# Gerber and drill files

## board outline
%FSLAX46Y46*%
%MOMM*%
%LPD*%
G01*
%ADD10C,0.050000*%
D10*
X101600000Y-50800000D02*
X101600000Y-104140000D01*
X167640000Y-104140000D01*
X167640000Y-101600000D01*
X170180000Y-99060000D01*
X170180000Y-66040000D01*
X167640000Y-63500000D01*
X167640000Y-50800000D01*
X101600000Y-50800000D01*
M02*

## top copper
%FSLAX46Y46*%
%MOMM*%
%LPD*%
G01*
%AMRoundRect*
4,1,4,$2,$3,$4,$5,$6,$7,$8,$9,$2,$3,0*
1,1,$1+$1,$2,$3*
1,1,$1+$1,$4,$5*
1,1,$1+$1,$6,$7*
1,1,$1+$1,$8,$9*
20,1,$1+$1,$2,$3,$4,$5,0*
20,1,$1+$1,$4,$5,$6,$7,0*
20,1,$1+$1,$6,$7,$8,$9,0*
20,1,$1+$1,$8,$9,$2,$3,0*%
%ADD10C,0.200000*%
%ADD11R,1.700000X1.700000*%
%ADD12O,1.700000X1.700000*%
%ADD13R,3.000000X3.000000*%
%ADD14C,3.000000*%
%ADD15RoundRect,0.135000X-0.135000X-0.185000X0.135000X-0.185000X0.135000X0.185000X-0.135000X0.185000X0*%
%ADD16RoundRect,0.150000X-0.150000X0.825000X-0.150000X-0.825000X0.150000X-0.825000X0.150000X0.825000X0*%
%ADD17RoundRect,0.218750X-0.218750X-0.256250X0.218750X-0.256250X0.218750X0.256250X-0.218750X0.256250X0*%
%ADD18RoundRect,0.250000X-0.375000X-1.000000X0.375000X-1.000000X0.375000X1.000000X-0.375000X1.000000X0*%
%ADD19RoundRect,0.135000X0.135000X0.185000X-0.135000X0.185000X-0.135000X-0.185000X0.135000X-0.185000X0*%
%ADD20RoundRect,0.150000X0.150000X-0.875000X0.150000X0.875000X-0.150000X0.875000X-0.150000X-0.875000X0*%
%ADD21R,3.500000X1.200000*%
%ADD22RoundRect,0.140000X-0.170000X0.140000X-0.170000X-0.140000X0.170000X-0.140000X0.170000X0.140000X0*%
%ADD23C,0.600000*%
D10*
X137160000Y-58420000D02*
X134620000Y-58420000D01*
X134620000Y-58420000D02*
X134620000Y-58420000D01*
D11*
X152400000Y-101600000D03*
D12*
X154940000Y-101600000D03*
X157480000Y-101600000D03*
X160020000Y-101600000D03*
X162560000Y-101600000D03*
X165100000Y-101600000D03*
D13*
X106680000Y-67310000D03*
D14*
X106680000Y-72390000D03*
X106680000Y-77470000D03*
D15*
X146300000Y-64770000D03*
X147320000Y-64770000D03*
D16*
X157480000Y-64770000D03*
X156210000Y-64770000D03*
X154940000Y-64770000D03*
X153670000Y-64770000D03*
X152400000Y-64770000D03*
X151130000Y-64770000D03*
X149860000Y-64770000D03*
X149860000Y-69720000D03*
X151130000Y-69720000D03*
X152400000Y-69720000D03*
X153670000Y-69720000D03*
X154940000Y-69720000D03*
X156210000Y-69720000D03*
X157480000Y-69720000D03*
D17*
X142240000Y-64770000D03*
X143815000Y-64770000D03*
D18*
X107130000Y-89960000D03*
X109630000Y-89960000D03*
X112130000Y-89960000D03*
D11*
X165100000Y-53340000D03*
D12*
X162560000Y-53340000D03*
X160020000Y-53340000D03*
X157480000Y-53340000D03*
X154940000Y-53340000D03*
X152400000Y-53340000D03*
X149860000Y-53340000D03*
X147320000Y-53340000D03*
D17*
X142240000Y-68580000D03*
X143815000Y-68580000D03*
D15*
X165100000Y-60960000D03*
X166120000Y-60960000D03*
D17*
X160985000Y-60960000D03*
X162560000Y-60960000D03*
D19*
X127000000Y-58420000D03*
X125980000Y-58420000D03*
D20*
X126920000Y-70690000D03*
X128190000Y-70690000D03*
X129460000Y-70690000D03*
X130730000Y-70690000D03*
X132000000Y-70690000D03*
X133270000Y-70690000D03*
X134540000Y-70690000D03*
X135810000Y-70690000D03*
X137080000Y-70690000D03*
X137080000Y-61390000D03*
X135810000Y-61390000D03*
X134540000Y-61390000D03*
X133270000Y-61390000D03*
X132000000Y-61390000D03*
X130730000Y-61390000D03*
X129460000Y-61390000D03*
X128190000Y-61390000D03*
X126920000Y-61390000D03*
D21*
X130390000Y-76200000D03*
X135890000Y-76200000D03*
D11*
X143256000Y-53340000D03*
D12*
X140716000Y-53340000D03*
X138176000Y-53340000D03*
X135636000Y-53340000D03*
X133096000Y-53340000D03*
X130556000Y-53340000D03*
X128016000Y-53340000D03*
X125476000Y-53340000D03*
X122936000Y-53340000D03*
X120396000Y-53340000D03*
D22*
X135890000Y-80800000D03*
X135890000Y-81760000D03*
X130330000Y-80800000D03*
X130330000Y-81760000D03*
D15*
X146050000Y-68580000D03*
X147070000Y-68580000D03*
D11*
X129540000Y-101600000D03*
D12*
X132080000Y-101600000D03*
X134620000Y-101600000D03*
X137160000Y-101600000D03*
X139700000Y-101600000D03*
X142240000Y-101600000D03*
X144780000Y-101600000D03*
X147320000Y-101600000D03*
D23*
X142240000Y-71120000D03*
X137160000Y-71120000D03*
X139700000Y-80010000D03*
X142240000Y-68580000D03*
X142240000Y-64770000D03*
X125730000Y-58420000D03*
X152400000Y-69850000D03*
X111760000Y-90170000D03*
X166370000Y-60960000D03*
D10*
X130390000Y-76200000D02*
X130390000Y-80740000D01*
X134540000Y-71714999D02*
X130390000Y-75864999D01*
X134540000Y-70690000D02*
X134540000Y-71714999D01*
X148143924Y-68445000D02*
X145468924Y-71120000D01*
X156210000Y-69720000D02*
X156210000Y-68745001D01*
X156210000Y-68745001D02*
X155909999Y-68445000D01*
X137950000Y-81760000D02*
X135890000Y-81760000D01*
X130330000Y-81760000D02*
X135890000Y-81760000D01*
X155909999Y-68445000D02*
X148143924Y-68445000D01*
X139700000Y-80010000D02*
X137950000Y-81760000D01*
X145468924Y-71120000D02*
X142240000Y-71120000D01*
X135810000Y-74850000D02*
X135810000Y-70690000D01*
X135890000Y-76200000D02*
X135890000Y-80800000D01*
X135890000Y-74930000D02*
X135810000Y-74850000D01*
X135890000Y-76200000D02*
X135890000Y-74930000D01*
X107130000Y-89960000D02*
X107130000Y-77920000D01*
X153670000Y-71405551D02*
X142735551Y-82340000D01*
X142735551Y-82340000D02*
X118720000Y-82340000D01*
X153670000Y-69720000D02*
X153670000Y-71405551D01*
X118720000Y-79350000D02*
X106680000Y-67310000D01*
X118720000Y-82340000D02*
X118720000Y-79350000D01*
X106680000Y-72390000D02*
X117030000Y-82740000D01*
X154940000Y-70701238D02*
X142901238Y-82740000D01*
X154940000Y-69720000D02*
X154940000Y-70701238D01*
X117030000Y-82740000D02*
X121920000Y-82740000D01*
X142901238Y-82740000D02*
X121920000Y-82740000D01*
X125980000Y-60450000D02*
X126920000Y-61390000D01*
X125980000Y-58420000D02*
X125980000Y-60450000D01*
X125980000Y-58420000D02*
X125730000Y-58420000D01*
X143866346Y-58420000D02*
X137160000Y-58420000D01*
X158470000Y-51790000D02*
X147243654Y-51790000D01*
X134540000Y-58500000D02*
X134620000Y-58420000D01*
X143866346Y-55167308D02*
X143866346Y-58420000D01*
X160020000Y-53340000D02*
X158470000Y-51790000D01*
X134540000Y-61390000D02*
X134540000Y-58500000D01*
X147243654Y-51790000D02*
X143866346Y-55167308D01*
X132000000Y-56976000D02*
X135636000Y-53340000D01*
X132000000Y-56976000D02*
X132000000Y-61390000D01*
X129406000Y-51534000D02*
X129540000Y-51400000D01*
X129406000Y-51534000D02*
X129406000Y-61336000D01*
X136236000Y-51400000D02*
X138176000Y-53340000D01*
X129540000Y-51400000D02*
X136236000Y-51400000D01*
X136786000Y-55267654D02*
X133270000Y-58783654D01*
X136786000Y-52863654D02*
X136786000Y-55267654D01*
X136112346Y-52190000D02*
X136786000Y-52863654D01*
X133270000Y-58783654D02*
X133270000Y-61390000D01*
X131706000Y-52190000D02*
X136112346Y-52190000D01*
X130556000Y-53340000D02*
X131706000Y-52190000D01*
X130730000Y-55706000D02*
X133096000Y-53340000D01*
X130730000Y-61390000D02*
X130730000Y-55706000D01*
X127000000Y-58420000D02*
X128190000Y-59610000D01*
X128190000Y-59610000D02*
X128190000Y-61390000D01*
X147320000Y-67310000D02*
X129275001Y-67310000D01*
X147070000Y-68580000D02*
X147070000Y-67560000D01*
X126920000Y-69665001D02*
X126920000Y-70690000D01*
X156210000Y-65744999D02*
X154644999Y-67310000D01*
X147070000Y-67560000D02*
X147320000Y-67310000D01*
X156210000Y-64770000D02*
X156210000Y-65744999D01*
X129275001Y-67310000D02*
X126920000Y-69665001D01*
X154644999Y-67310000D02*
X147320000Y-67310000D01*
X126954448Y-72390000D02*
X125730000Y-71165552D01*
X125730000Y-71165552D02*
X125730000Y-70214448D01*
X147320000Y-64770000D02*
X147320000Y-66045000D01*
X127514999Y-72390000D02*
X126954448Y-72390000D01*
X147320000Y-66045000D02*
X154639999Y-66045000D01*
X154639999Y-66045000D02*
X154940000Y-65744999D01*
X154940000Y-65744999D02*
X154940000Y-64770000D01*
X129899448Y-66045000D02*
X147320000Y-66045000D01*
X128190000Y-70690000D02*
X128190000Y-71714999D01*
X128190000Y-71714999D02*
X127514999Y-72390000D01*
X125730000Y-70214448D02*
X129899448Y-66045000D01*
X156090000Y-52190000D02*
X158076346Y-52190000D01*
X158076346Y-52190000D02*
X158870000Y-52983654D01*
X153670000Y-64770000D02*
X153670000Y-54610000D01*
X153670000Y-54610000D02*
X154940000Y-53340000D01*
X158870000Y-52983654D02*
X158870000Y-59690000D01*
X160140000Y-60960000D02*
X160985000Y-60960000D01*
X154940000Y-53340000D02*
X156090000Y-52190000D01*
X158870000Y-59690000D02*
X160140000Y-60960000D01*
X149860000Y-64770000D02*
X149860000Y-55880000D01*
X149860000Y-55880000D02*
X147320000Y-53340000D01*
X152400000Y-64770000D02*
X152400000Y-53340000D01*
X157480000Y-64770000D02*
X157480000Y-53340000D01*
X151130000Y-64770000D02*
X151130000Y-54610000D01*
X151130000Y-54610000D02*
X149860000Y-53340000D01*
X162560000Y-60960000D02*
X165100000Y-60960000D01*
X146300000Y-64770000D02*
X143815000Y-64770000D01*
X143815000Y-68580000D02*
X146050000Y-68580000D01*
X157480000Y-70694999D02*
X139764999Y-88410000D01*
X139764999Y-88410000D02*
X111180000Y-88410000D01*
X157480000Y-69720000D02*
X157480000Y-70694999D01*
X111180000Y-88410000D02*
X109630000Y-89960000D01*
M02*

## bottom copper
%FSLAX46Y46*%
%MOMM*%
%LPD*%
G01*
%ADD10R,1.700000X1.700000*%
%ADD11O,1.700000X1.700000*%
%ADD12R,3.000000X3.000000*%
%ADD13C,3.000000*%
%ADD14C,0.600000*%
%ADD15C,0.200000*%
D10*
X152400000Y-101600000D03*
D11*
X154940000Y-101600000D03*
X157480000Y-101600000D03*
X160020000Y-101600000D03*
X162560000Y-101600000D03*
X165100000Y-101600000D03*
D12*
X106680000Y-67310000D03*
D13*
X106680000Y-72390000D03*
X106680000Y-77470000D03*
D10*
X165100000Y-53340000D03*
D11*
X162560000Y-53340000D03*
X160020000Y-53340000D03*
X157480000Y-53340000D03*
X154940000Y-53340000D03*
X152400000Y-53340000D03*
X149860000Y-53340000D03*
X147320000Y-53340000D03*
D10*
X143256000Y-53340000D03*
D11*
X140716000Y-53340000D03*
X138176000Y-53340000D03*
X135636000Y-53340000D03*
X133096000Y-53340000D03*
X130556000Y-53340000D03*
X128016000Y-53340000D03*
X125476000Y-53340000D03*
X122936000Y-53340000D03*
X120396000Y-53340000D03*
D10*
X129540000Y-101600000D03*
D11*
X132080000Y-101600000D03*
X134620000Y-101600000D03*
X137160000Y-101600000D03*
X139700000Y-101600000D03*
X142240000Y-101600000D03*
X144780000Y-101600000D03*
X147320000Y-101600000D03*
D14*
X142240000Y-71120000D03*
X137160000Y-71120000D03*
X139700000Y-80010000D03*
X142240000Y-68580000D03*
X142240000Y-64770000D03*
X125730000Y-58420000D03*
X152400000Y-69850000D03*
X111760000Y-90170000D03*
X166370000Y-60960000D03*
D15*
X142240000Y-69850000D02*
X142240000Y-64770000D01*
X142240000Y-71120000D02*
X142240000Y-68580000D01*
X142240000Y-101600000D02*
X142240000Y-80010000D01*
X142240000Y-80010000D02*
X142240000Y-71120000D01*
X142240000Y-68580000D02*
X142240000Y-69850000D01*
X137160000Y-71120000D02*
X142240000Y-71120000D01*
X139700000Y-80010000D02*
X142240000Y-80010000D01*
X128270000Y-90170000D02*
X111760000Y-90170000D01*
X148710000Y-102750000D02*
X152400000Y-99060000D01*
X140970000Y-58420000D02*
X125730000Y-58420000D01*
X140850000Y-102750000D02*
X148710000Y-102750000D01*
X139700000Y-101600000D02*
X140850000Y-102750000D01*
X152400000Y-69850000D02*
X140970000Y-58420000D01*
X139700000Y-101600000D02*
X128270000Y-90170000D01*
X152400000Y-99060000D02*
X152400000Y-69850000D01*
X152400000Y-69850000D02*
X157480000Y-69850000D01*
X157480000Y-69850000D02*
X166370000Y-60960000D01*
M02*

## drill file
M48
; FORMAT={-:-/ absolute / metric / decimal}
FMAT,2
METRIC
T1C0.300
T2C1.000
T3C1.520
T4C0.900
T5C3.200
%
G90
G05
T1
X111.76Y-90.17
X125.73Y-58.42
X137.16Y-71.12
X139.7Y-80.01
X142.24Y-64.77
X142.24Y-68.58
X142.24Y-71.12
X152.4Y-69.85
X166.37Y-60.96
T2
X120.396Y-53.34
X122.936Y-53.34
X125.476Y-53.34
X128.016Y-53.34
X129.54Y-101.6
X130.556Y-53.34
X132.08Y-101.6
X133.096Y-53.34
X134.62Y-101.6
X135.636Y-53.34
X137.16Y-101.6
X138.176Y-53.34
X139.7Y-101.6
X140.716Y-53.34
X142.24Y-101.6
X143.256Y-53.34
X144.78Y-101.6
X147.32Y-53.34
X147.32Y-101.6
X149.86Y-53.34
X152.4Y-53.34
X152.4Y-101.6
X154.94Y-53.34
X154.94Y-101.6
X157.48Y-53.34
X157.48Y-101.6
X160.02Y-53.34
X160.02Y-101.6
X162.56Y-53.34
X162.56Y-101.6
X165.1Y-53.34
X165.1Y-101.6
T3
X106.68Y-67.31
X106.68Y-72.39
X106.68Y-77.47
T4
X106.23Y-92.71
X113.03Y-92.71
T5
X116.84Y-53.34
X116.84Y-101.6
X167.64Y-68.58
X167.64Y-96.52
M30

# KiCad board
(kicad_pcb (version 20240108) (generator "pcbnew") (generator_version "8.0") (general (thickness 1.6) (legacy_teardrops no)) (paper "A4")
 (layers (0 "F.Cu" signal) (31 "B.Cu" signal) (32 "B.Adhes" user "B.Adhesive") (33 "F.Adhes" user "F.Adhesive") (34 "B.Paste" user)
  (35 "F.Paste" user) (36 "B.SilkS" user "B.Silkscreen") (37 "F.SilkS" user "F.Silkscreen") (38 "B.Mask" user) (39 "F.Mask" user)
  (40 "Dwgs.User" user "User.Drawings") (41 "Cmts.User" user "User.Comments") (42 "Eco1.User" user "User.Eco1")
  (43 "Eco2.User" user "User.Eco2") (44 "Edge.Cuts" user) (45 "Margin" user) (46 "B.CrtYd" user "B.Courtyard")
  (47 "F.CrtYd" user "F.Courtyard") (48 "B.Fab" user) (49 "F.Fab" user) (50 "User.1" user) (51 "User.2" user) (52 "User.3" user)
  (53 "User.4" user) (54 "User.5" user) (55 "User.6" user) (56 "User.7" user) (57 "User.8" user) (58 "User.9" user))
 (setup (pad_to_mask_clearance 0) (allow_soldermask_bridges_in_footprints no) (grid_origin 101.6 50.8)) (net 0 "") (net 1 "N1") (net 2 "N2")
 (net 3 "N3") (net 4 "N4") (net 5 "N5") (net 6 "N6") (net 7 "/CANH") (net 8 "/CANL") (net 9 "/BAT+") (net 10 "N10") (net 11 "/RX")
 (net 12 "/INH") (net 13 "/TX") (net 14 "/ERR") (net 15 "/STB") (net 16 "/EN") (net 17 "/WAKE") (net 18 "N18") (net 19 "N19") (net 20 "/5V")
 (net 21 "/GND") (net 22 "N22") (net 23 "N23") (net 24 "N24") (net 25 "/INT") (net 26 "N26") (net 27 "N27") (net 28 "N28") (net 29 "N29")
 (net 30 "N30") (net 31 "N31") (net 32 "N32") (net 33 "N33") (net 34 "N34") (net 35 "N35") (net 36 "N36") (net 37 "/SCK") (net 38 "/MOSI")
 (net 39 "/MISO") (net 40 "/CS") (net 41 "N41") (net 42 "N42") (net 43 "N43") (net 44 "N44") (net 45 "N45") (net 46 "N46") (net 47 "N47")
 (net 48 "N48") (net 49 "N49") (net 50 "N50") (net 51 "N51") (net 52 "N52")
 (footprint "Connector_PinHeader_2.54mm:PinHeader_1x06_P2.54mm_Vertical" (layer "F.Cu") (at 152.4 101.6 90)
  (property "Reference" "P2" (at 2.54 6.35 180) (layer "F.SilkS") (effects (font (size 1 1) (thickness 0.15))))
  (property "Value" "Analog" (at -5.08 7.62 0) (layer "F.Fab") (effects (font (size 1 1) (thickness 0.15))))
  (pad "1" thru_hole rect (at 0 0 90) (size 1.7 1.7) (drill 1) (layers "*.Cu" "*.Mask") (remove_unused_layers no) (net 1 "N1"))
  (pad "2" thru_hole oval (at 0 2.54 90) (size 1.7 1.7) (drill 1) (layers "*.Cu" "*.Mask") (remove_unused_layers no) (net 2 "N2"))
  (pad "3" thru_hole oval (at 0 5.08 90) (size 1.7 1.7) (drill 1) (layers "*.Cu" "*.Mask") (remove_unused_layers no) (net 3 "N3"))
  (pad "4" thru_hole oval (at 0 7.62 90) (size 1.7 1.7) (drill 1) (layers "*.Cu" "*.Mask") (remove_unused_layers no) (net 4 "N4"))
  (pad "5" thru_hole oval (at 0 10.16 90) (size 1.7 1.7) (drill 1) (layers "*.Cu" "*.Mask") (remove_unused_layers no) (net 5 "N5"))
  (pad "6" thru_hole oval (at 0 12.7 90) (size 1.7 1.7) (drill 1) (layers "*.Cu" "*.Mask") (remove_unused_layers no) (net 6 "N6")))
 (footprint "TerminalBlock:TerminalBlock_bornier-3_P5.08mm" (layer "F.Cu") (at 106.68 67.31 -90)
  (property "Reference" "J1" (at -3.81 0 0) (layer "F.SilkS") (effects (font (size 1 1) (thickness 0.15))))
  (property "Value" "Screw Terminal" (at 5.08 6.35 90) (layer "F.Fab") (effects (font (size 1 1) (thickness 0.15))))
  (pad "1" thru_hole rect (at 0 0 270) (size 3 3) (drill 1.52) (layers "*.Cu" "*.Mask") (remove_unused_layers no) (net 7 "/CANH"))
  (pad "2" thru_hole circle (at 5.08 0 270) (size 3 3) (drill 1.52) (layers "*.Cu" "*.Mask") (remove_unused_layers no) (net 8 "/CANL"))
  (pad "3" thru_hole circle (at 10.16 0 270) (size 3 3) (drill 1.52) (layers "*.Cu" "*.Mask") (remove_unused_layers no) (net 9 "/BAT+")))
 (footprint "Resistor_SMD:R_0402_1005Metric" (layer "F.Cu") (at 146.81 64.77)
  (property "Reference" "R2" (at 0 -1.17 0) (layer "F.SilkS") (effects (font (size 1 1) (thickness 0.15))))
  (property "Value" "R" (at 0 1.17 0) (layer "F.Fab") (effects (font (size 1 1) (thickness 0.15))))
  (pad "1" smd roundrect (at -0.51 0) (size 0.54 0.64) (layers "F.Cu" "F.Paste" "F.Mask") (roundrect_rratio 0.25) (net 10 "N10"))
  (pad "2" smd roundrect (at 0.51 0) (size 0.54 0.64) (layers "F.Cu" "F.Paste" "F.Mask") (roundrect_rratio 0.25) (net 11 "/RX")))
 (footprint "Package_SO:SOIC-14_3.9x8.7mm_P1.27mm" (layer "F.Cu") (at 153.67 67.245 -90)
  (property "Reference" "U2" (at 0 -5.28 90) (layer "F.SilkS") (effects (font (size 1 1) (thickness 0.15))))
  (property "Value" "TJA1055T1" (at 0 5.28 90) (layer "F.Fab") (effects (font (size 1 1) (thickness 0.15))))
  (pad "1" smd roundrect (at -2.475 -3.81 270) (size 1.95 0.6) (layers "F.Cu" "F.Paste" "F.Mask") (roundrect_rratio 0.25) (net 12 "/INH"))
  (pad "2" smd roundrect (at -2.475 -2.54 270) (size 1.95 0.6) (layers "F.Cu" "F.Paste" "F.Mask") (roundrect_rratio 0.25) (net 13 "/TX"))
  (pad "3" smd roundrect (at -2.475 -1.27 270) (size 1.95 0.6) (layers "F.Cu" "F.Paste" "F.Mask") (roundrect_rratio 0.25) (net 11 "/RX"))
  (pad "4" smd roundrect (at -2.475 0 270) (size 1.95 0.6) (layers "F.Cu" "F.Paste" "F.Mask") (roundrect_rratio 0.25) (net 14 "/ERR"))
  (pad "5" smd roundrect (at -2.475 1.27 270) (size 1.95 0.6) (layers "F.Cu" "F.Paste" "F.Mask") (roundrect_rratio 0.25) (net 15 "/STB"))
  (pad "6" smd roundrect (at -2.475 2.54 270) (size 1.95 0.6) (layers "F.Cu" "F.Paste" "F.Mask") (roundrect_rratio 0.25) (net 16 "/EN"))
  (pad "7" smd roundrect (at -2.475 3.81 270) (size 1.95 0.6) (layers "F.Cu" "F.Paste" "F.Mask") (roundrect_rratio 0.25) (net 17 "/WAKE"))
  (pad "8" smd roundrect (at 2.475 3.81 270) (size 1.95 0.6) (layers "F.Cu" "F.Paste" "F.Mask") (roundrect_rratio 0.25) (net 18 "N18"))
  (pad "9" smd roundrect (at 2.475 2.54 270) (size 1.95 0.6) (layers "F.Cu" "F.Paste" "F.Mask") (roundrect_rratio 0.25) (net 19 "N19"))
  (pad "10" smd roundrect (at 2.475 1.27 270) (size 1.95 0.6) (layers "F.Cu" "F.Paste" "F.Mask") (roundrect_rratio 0.25) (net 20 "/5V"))
  (pad "11" smd roundrect (at 2.475 0 270) (size 1.95 0.6) (layers "F.Cu" "F.Paste" "F.Mask") (roundrect_rratio 0.25) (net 7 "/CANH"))
  (pad "12" smd roundrect (at 2.475 -1.27 270) (size 1.95 0.6) (layers "F.Cu" "F.Paste" "F.Mask") (roundrect_rratio 0.25) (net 8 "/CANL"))
  (pad "13" smd roundrect (at 2.475 -2.54 270) (size 1.95 0.6) (layers "F.Cu" "F.Paste" "F.Mask") (roundrect_rratio 0.25) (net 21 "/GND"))
  (pad "14" smd roundrect (at 2.475 -3.81 270) (size 1.95 0.6) (layers "F.Cu" "F.Paste" "F.Mask") (roundrect_rratio 0.25) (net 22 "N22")))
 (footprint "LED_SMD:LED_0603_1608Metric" (layer "F.Cu") (at 143.0275 64.77)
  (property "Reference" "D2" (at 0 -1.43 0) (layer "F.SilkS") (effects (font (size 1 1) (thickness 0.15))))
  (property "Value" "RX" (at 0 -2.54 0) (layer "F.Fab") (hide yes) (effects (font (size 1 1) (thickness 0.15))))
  (pad "1" smd roundrect (at -0.7875 0) (size 0.875 0.95) (layers "F.Cu" "F.Paste" "F.Mask") (roundrect_rratio 0.25) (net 21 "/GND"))
  (pad "2" smd roundrect (at 0.7875 0) (size 0.875 0.95) (layers "F.Cu" "F.Paste" "F.Mask") (roundrect_rratio 0.25) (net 10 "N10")))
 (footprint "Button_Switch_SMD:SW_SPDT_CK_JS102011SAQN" (layer "F.Cu") (at 109.63 92.71)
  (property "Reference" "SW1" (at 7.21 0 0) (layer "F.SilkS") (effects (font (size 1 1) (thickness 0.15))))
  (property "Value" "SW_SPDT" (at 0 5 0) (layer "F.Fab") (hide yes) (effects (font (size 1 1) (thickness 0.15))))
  (pad "" np_thru_hole circle (at -3.4 0) (size 0.9 0.9) (drill 0.9) (layers "*.Cu" "*.Mask"))
  (pad "" np_thru_hole circle (at 3.4 0) (size 0.9 0.9) (drill 0.9) (layers "*.Cu" "*.Mask"))
  (pad "1" smd roundrect (at -2.5 -2.75) (size 1.25 2.5) (layers "F.Cu" "F.Paste" "F.Mask") (roundrect_rratio 0.2) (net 9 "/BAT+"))
  (pad "2" smd roundrect (at 0 -2.75) (size 1.25 2.5) (layers "F.Cu" "F.Paste" "F.Mask") (roundrect_rratio 0.2) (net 22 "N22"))
  (pad "3" smd roundrect (at 2.5 -2.75) (size 1.25 2.5) (layers "F.Cu" "F.Paste" "F.Mask") (roundrect_rratio 0.2) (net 20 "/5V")))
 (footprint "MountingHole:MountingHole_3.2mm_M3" (layer "F.Cu") (at 116.84 53.34)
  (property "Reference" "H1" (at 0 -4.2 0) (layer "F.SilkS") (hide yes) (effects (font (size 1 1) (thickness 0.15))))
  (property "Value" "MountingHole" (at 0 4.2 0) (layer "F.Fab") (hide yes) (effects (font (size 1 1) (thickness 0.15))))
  (pad "" np_thru_hole circle (at 0 0) (size 3.2 3.2) (drill 3.2) (layers "*.Cu" "*.Mask")))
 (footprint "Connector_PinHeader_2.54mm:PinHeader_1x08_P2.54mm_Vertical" (layer "F.Cu") (at 165.1 53.34 -90)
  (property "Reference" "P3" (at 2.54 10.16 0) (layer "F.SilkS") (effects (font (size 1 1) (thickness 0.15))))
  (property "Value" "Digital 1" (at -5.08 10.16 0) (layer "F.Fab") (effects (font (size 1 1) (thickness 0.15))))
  (pad "1" thru_hole rect (at 0 0 270) (size 1.7 1.7) (drill 1) (layers "*.Cu" "*.Mask") (remove_unused_layers no) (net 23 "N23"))
  (pad "2" thru_hole oval (at 0 2.54 270) (size 1.7 1.7) (drill 1) (layers "*.Cu" "*.Mask") (remove_unused_layers no) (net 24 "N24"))
  (pad "3" thru_hole oval (at 0 5.08 270) (size 1.7 1.7) (drill 1) (layers "*.Cu" "*.Mask") (remove_unused_layers no) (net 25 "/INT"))
  (pad "4" thru_hole oval (at 0 7.62 270) (size 1.7 1.7) (drill 1) (layers "*.Cu" "*.Mask") (remove_unused_layers no) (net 12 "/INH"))
  (pad "5" thru_hole oval (at 0 10.16 270) (size 1.7 1.7) (drill 1) (layers "*.Cu" "*.Mask") (remove_unused_layers no) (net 14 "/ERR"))
  (pad "6" thru_hole oval (at 0 12.7 270) (size 1.7 1.7) (drill 1) (layers "*.Cu" "*.Mask") (remove_unused_layers no) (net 15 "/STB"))
  (pad "7" thru_hole oval (at 0 15.24 270) (size 1.7 1.7) (drill 1) (layers "*.Cu" "*.Mask") (remove_unused_layers no) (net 16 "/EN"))
  (pad "8" thru_hole oval (at 0 17.78 270) (size 1.7 1.7) (drill 1) (layers "*.Cu" "*.Mask") (remove_unused_layers no) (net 17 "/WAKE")))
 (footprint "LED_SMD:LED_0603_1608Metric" (layer "F.Cu") (at 143.0275 68.58)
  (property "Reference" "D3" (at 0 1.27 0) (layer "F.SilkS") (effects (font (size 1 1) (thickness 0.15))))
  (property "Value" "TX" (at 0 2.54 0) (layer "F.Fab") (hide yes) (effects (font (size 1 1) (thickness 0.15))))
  (pad "1" smd roundrect (at -0.7875 0) (size 0.875 0.95) (layers "F.Cu" "F.Paste" "F.Mask") (roundrect_rratio 0.25) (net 21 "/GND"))
  (pad "2" smd roundrect (at 0.7875 0) (size 0.875 0.95) (layers "F.Cu" "F.Paste" "F.Mask") (roundrect_rratio 0.25) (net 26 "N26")))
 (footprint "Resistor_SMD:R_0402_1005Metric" (layer "F.Cu") (at 165.61 60.96)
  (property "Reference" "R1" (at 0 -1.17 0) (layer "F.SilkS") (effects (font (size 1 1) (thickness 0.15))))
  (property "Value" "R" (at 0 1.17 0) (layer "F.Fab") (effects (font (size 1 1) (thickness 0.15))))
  (pad "1" smd roundrect (at -0.51 0) (size 0.54 0.64) (layers "F.Cu" "F.Paste" "F.Mask") (roundrect_rratio 0.25) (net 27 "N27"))
  (pad "2" smd roundrect (at 0.51 0) (size 0.54 0.64) (layers "F.Cu" "F.Paste" "F.Mask") (roundrect_rratio 0.25) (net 20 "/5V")))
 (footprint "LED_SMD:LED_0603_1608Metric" (layer "F.Cu") (at 161.7725 60.96)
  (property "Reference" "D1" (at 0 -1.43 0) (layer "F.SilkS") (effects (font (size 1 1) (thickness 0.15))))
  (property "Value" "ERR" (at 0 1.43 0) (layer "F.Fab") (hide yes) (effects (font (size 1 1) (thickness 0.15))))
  (pad "1" smd roundrect (at -0.7875 0) (size 0.875 0.95) (layers "F.Cu" "F.Paste" "F.Mask") (roundrect_rratio 0.25) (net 14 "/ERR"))
  (pad "2" smd roundrect (at 0.7875 0) (size 0.875 0.95) (layers "F.Cu" "F.Paste" "F.Mask") (roundrect_rratio 0.25) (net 27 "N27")))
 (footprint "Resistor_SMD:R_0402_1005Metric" (layer "F.Cu") (at 126.49 58.42 180)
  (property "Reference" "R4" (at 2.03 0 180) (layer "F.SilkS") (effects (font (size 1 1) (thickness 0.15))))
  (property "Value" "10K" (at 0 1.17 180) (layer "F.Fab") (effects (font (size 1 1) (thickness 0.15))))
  (pad "1" smd roundrect (at -0.51 0 180) (size 0.54 0.64) (layers "F.Cu" "F.Paste" "F.Mask") (roundrect_rratio 0.25) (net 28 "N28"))
  (pad "2" smd roundrect (at 0.51 0 180) (size 0.54 0.64) (layers "F.Cu" "F.Paste" "F.Mask") (roundrect_rratio 0.25) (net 20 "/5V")))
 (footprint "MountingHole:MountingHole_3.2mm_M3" (layer "F.Cu") (at 167.64 68.58)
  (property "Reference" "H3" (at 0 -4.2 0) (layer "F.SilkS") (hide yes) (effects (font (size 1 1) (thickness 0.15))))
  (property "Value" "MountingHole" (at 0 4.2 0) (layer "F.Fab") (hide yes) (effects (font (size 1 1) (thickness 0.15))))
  (pad "" np_thru_hole circle (at 0 0) (size 3.2 3.2) (drill 3.2) (layers "*.Cu" "*.Mask")))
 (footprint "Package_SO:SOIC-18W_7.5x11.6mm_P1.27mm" (layer "F.Cu") (at 132 66.04 90)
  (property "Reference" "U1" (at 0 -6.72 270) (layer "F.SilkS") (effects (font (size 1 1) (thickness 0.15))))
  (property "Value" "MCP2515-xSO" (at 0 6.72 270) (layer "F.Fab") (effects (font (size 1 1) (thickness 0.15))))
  (pad "1" smd roundrect (at -4.65 -5.08 90) (size 2.05 0.6) (layers "F.Cu" "F.Paste" "F.Mask") (roundrect_rratio 0.25) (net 13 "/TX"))
  (pad "2" smd roundrect (at -4.65 -3.81 90) (size 2.05 0.6) (layers "F.Cu" "F.Paste" "F.Mask") (roundrect_rratio 0.25) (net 11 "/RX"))
  (pad "3" smd roundrect (at -4.65 -2.54 90) (size 2.05 0.6) (layers "F.Cu" "F.Paste" "F.Mask") (roundrect_rratio 0.25) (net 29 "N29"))
  (pad "4" smd roundrect (at -4.65 -1.27 90) (size 2.05 0.6) (layers "F.Cu" "F.Paste" "F.Mask") (roundrect_rratio 0.25) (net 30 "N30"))
  (pad "5" smd roundrect (at -4.65 0 90) (size 2.05 0.6) (layers "F.Cu" "F.Paste" "F.Mask") (roundrect_rratio 0.25) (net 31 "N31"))
  (pad "6" smd roundrect (at -4.65 1.27 90) (size 2.05 0.6) (layers "F.Cu" "F.Paste" "F.Mask") (roundrect_rratio 0.25) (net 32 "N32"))
  (pad "7" smd roundrect (at -4.65 2.54 90) (size 2.05 0.6) (layers "F.Cu" "F.Paste" "F.Mask") (roundrect_rratio 0.25) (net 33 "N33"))
  (pad "8" smd roundrect (at -4.65 3.81 90) (size 2.05 0.6) (layers "F.Cu" "F.Paste" "F.Mask") (roundrect_rratio 0.25) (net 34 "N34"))
  (pad "9" smd roundrect (at -4.65 5.08 90) (size 2.05 0.6) (layers "F.Cu" "F.Paste" "F.Mask") (roundrect_rratio 0.25) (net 21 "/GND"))
  (pad "10" smd roundrect (at 4.65 5.08 90) (size 2.05 0.6) (layers "F.Cu" "F.Paste" "F.Mask") (roundrect_rratio 0.25) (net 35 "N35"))
  (pad "11" smd roundrect (at 4.65 3.81 90) (size 2.05 0.6) (layers "F.Cu" "F.Paste" "F.Mask") (roundrect_rratio 0.25) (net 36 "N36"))
  (pad "12" smd roundrect (at 4.65 2.54 90) (size 2.05 0.6) (layers "F.Cu" "F.Paste" "F.Mask") (roundrect_rratio 0.25) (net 25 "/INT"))
  (pad "13" smd roundrect (at 4.65 1.27 90) (size 2.05 0.6) (layers "F.Cu" "F.Paste" "F.Mask") (roundrect_rratio 0.25) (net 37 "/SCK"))
  (pad "14" smd roundrect (at 4.65 0 90) (size 2.05 0.6) (layers "F.Cu" "F.Paste" "F.Mask") (roundrect_rratio 0.25) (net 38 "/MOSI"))
  (pad "15" smd roundrect (at 4.65 -1.27 90) (size 2.05 0.6) (layers "F.Cu" "F.Paste" "F.Mask") (roundrect_rratio 0.25) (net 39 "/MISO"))
  (pad "16" smd roundrect (at 4.65 -2.54 90) (size 2.05 0.6) (layers "F.Cu" "F.Paste" "F.Mask") (roundrect_rratio 0.25) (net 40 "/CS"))
  (pad "17" smd roundrect (at 4.65 -3.81 90) (size 2.05 0.6) (layers "F.Cu" "F.Paste" "F.Mask") (roundrect_rratio 0.25) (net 28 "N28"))
  (pad "18" smd roundrect (at 4.65 -5.08 90) (size 2.05 0.6) (layers "F.Cu" "F.Paste" "F.Mask") (roundrect_rratio 0.25) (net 20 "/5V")))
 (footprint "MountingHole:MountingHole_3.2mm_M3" (layer "F.Cu") (at 116.84 101.6)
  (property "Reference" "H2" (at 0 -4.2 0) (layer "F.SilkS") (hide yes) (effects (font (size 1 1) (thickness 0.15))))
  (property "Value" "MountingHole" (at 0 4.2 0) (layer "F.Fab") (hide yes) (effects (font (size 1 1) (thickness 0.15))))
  (pad "" np_thru_hole circle (at 0 0) (size 3.2 3.2) (drill 3.2) (layers "*.Cu" "*.Mask")))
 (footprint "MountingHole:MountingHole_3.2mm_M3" (layer "F.Cu") (at 167.64 96.52)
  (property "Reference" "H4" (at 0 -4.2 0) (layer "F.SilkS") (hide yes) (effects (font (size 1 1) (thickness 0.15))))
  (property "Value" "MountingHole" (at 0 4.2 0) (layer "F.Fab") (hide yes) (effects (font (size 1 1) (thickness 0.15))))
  (pad "" np_thru_hole circle (at 0 0) (size 3.2 3.2) (drill 3.2) (layers "*.Cu" "*.Mask")))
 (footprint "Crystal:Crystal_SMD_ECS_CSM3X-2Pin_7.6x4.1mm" (layer "F.Cu") (at 133.14 76.2)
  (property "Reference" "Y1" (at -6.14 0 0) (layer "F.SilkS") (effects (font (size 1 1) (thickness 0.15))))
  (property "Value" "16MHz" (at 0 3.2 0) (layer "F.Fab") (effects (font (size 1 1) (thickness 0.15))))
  (pad "1" smd rect (at -2.75 0) (size 3.5 1.2) (layers "F.Cu" "F.Paste" "F.Mask") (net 33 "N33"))
  (pad "2" smd rect (at 2.75 0) (size 3.5 1.2) (layers "F.Cu" "F.Paste" "F.Mask") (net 34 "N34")))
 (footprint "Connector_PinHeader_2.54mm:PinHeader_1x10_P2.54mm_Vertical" (layer "F.Cu") (at 143.256 53.34 -90)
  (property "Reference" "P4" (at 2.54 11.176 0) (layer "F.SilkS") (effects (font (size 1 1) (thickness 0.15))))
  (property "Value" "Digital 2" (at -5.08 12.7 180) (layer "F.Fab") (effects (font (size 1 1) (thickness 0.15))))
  (pad "1" thru_hole rect (at 0 0 270) (size 1.7 1.7) (drill 1) (layers "*.Cu" "*.Mask") (remove_unused_layers no) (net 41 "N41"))
  (pad "2" thru_hole oval (at 0 2.54 270) (size 1.7 1.7) (drill 1) (layers "*.Cu" "*.Mask") (remove_unused_layers no) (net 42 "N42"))
  (pad "3" thru_hole oval (at 0 5.08 270) (size 1.7 1.7) (drill 1) (layers "*.Cu" "*.Mask") (remove_unused_layers no) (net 40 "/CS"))
  (pad "4" thru_hole oval (at 0 7.62 270) (size 1.7 1.7) (drill 1) (layers "*.Cu" "*.Mask") (remove_unused_layers no) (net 38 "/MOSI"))
  (pad "5" thru_hole oval (at 0 10.16 270) (size 1.7 1.7) (drill 1) (layers "*.Cu" "*.Mask") (remove_unused_layers no) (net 39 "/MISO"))
  (pad "6" thru_hole oval (at 0 12.7 270) (size 1.7 1.7) (drill 1) (layers "*.Cu" "*.Mask") (remove_unused_layers no) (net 37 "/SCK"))
  (pad "7" thru_hole oval (at 0 15.24 270) (size 1.7 1.7) (drill 1) (layers "*.Cu" "*.Mask") (remove_unused_layers no) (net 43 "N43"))
  (pad "8" thru_hole oval (at 0 17.78 270) (size 1.7 1.7) (drill 1) (layers "*.Cu" "*.Mask") (remove_unused_layers no) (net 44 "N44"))
  (pad "9" thru_hole oval (at 0 20.32 270) (size 1.7 1.7) (drill 1) (layers "*.Cu" "*.Mask") (remove_unused_layers no) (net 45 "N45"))
  (pad "10" thru_hole oval (at 0 22.86 270) (size 1.7 1.7) (drill 1) (layers "*.Cu" "*.Mask") (remove_unused_layers no) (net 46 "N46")))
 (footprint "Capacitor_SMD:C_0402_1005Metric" (layer "F.Cu") (at 135.89 81.28 -90)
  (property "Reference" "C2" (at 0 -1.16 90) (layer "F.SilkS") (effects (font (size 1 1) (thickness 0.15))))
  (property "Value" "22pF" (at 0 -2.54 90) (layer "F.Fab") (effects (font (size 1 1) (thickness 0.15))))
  (pad "1" smd roundrect (at -0.48 0 270) (size 0.56 0.62) (layers "F.Cu" "F.Paste" "F.Mask") (roundrect_rratio 0.25) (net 34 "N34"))
  (pad "2" smd roundrect (at 0.48 0 270) (size 0.56 0.62) (layers "F.Cu" "F.Paste" "F.Mask") (roundrect_rratio 0.25) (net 21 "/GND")))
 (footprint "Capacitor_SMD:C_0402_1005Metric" (layer "F.Cu") (at 130.33 81.28 -90)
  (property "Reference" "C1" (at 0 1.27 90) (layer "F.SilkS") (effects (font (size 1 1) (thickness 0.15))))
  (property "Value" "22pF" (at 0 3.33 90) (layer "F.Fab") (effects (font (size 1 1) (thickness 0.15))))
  (pad "1" smd roundrect (at -0.48 0 270) (size 0.56 0.62) (layers "F.Cu" "F.Paste" "F.Mask") (roundrect_rratio 0.25) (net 33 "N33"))
  (pad "2" smd roundrect (at 0.48 0 270) (size 0.56 0.62) (layers "F.Cu" "F.Paste" "F.Mask") (roundrect_rratio 0.25) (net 21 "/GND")))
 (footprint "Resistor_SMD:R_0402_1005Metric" (layer "F.Cu") (at 146.56 68.58)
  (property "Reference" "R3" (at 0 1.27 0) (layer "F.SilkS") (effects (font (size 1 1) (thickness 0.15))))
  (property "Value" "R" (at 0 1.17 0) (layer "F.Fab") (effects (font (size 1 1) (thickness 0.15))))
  (pad "1" smd roundrect (at -0.51 0) (size 0.54 0.64) (layers "F.Cu" "F.Paste" "F.Mask") (roundrect_rratio 0.25) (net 26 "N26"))
  (pad "2" smd roundrect (at 0.51 0) (size 0.54 0.64) (layers "F.Cu" "F.Paste" "F.Mask") (roundrect_rratio 0.25) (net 13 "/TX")))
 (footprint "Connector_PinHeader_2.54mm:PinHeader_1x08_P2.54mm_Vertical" (layer "F.Cu") (at 129.54 101.6 90)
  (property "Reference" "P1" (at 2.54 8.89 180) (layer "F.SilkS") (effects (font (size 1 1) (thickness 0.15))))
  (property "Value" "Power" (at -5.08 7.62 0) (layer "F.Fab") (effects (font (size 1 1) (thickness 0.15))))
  (pad "1" thru_hole rect (at 0 0 90) (size 1.7 1.7) (drill 1) (layers "*.Cu" "*.Mask") (remove_unused_layers no) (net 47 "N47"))
  (pad "2" thru_hole oval (at 0 2.54 90) (size 1.7 1.7) (drill 1) (layers "*.Cu" "*.Mask") (remove_unused_layers no) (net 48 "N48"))
  (pad "3" thru_hole oval (at 0 5.08 90) (size 1.7 1.7) (drill 1) (layers "*.Cu" "*.Mask") (remove_unused_layers no) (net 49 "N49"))
  (pad "4" thru_hole oval (at 0 7.62 90) (size 1.7 1.7) (drill 1) (layers "*.Cu" "*.Mask") (remove_unused_layers no) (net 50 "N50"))
  (pad "5" thru_hole oval (at 0 10.16 90) (size 1.7 1.7) (drill 1) (layers "*.Cu" "*.Mask") (remove_unused_layers no) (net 20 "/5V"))
  (pad "6" thru_hole oval (at 0 12.7 90) (size 1.7 1.7) (drill 1) (layers "*.Cu" "*.Mask") (remove_unused_layers no) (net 21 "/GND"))
  (pad "7" thru_hole oval (at 0 15.24 90) (size 1.7 1.7) (drill 1) (layers "*.Cu" "*.Mask") (remove_unused_layers no) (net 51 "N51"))
  (pad "8" thru_hole oval (at 0 17.78 90) (size 1.7 1.7) (drill 1) (layers "*.Cu" "*.Mask") (remove_unused_layers no) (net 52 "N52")))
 (gr_line (start 137.16 58.42) (end 134.62 58.42) (stroke (width 0.2) (type default)) (layer "F.Cu") (net 25))
 (gr_line (start 134.62 58.42) (end 134.62 58.42) (stroke (width 0.2) (type default)) (layer "F.Cu") (net 25))
 (gr_poly
  (pts (xy 101.6 50.8) (xy 101.6 104.14) (xy 167.64 104.14) (xy 167.64 101.6) (xy 170.18 99.06) (xy 170.18 66.04) (xy 167.64 63.5)
   (xy 167.64 50.8))
  (stroke (width 0.05) (type solid)) (fill none) (layer "Edge.Cuts"))
 (segment (start 130.39 76.2) (end 130.39 80.74) (width 0.2) (layer "F.Cu") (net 33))
 (segment (start 134.54 71.714999) (end 130.39 75.864999) (width 0.2) (layer "F.Cu") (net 33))
 (segment (start 134.54 70.69) (end 134.54 71.714999) (width 0.2) (layer "F.Cu") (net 33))
 (segment (start 148.143924 68.445) (end 145.468924 71.12) (width 0.2) (layer "F.Cu") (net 21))
 (segment (start 156.21 69.72) (end 156.21 68.745001) (width 0.2) (layer "F.Cu") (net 21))
 (segment (start 156.21 68.745001) (end 155.909999 68.445) (width 0.2) (layer "F.Cu") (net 21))
 (segment (start 137.95 81.76) (end 135.89 81.76) (width 0.2) (layer "F.Cu") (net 21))
 (segment (start 130.33 81.76) (end 135.89 81.76) (width 0.2) (layer "F.Cu") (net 21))
 (segment (start 155.909999 68.445) (end 148.143924 68.445) (width 0.2) (layer "F.Cu") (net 21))
 (segment (start 139.7 80.01) (end 137.95 81.76) (width 0.2) (layer "F.Cu") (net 21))
 (segment (start 145.468924 71.12) (end 142.24 71.12) (width 0.2) (layer "F.Cu") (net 21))
 (via (at 142.24 71.12) (size 0.6) (drill 0.3) (layers "F.Cu" "B.Cu") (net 21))
 (via (at 137.16 71.12) (size 0.6) (drill 0.3) (layers "F.Cu" "B.Cu") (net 21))
 (via (at 139.7 80.01) (size 0.6) (drill 0.3) (layers "F.Cu" "B.Cu") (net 21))
 (via (at 142.24 68.58) (size 0.6) (drill 0.3) (layers "F.Cu" "B.Cu") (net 21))
 (via (at 142.24 64.77) (size 0.6) (drill 0.3) (layers "F.Cu" "B.Cu") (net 21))
 (segment (start 142.24 69.85) (end 142.24 64.77) (width 0.2) (layer "B.Cu") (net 21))
 (segment (start 142.24 71.12) (end 142.24 68.58) (width 0.2) (layer "B.Cu") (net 21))
 (segment (start 142.24 101.6) (end 142.24 80.01) (width 0.2) (layer "B.Cu") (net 21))
 (segment (start 142.24 80.01) (end 142.24 71.12) (width 0.2) (layer "B.Cu") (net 21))
 (segment (start 142.24 68.58) (end 142.24 69.85) (width 0.2) (layer "B.Cu") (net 21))
 (segment (start 137.16 71.12) (end 142.24 71.12) (width 0.2) (layer "B.Cu") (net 21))
 (segment (start 139.7 80.01) (end 142.24 80.01) (width 0.2) (layer "B.Cu") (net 21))
 (segment (start 135.81 74.85) (end 135.81 70.69) (width 0.2) (layer "F.Cu") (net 34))
 (segment (start 135.89 76.2) (end 135.89 80.8) (width 0.2) (layer "F.Cu") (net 34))
 (segment (start 135.89 74.93) (end 135.81 74.85) (width 0.2) (layer "F.Cu") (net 34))
 (segment (start 135.89 76.2) (end 135.89 74.93) (width 0.2) (layer "F.Cu") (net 34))
 (segment (start 107.13 89.96) (end 107.13 77.92) (width 0.2) (layer "F.Cu") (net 9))
 (segment (start 153.67 71.405551) (end 142.735551 82.34) (width 0.2) (layer "F.Cu") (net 7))
 (segment (start 142.735551 82.34) (end 118.72 82.34) (width 0.2) (layer "F.Cu") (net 7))
 (segment (start 153.67 69.72) (end 153.67 71.405551) (width 0.2) (layer "F.Cu") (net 7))
 (segment (start 118.72 79.35) (end 106.68 67.31) (width 0.2) (layer "F.Cu") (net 7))
 (segment (start 118.72 82.34) (end 118.72 79.35) (width 0.2) (layer "F.Cu") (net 7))
 (segment (start 106.68 72.39) (end 117.03 82.74) (width 0.2) (layer "F.Cu") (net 8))
 (segment (start 154.94 70.701238) (end 142.901238 82.74) (width 0.2) (layer "F.Cu") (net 8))
 (segment (start 154.94 69.72) (end 154.94 70.701238) (width 0.2) (layer "F.Cu") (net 8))
 (segment (start 117.03 82.74) (end 121.92 82.74) (width 0.2) (layer "F.Cu") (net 8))
 (segment (start 142.901238 82.74) (end 121.92 82.74) (width 0.2) (layer "F.Cu") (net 8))
 (segment (start 125.98 60.45) (end 126.92 61.39) (width 0.2) (layer "F.Cu") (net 20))
 (segment (start 125.98 58.42) (end 125.98 60.45) (width 0.2) (layer "F.Cu") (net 20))
 (segment (start 125.98 58.42) (end 125.73 58.42) (width 0.2) (layer "F.Cu") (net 20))
 (via (at 125.73 58.42) (size 0.6) (drill 0.3) (layers "F.Cu" "B.Cu") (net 20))
 (via (at 152.4 69.85) (size 0.6) (drill 0.3) (layers "F.Cu" "B.Cu") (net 20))
 (via (at 111.76 90.17) (size 0.6) (drill 0.3) (layers "F.Cu" "B.Cu") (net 20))
 (via (at 166.37 60.96) (size 0.6) (drill 0.3) (layers "F.Cu" "B.Cu") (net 20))
 (segment (start 128.27 90.17) (end 111.76 90.17) (width 0.2) (layer "B.Cu") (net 20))
 (segment (start 148.71 102.75) (end 152.4 99.06) (width 0.2) (layer "B.Cu") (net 20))
 (segment (start 140.97 58.42) (end 125.73 58.42) (width 0.2) (layer "B.Cu") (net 20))
 (segment (start 140.85 102.75) (end 148.71 102.75) (width 0.2) (layer "B.Cu") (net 20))
 (segment (start 139.7 101.6) (end 140.85 102.75) (width 0.2) (layer "B.Cu") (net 20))
 (segment (start 152.4 69.85) (end 140.97 58.42) (width 0.2) (layer "B.Cu") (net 20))
 (segment (start 139.7 101.6) (end 128.27 90.17) (width 0.2) (layer "B.Cu") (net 20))
 (segment (start 152.4 99.06) (end 152.4 69.85) (width 0.2) (layer "B.Cu") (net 20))
 (segment (start 152.4 69.85) (end 157.48 69.85) (width 0.2) (layer "B.Cu") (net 20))
 (segment (start 157.48 69.85) (end 166.37 60.96) (width 0.2) (layer "B.Cu") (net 20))
 (segment (start 143.866346 58.42) (end 137.16 58.42) (width 0.2) (layer "F.Cu") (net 25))
 (segment (start 158.47 51.79) (end 147.243654 51.79) (width 0.2) (layer "F.Cu") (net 25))
 (segment (start 134.54 58.5) (end 134.62 58.42) (width 0.2) (layer "F.Cu") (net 25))
 (segment (start 143.866346 55.167308) (end 143.866346 58.42) (width 0.2) (layer "F.Cu") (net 25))
 (segment (start 160.02 53.34) (end 158.47 51.79) (width 0.2) (layer "F.Cu") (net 25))
 (segment (start 134.54 61.39) (end 134.54 58.5) (width 0.2) (layer "F.Cu") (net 25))
 (segment (start 147.243654 51.79) (end 143.866346 55.167308) (width 0.2) (layer "F.Cu") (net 25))
 (segment (start 132 56.976) (end 135.636 53.34) (width 0.2) (layer "F.Cu") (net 38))
 (segment (start 132 56.976) (end 132 61.39) (width 0.2) (layer "F.Cu") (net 38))
 (segment (start 129.406 51.534) (end 129.54 51.4) (width 0.2) (layer "F.Cu") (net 40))
 (segment (start 129.406 51.534) (end 129.406 61.336) (width 0.2) (layer "F.Cu") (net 40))
 (segment (start 136.236 51.4) (end 138.176 53.34) (width 0.2) (layer "F.Cu") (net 40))
 (segment (start 129.54 51.4) (end 136.236 51.4) (width 0.2) (layer "F.Cu") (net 40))
 (segment (start 136.786 55.267654) (end 133.27 58.783654) (width 0.2) (layer "F.Cu") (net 37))
 (segment (start 136.786 52.863654) (end 136.786 55.267654) (width 0.2) (layer "F.Cu") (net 37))
 (segment (start 136.112346 52.19) (end 136.786 52.863654) (width 0.2) (layer "F.Cu") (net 37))
 (segment (start 133.27 58.783654) (end 133.27 61.39) (width 0.2) (layer "F.Cu") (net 37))
 (segment (start 131.706 52.19) (end 136.112346 52.19) (width 0.2) (layer "F.Cu") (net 37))
 (segment (start 130.556 53.34) (end 131.706 52.19) (width 0.2) (layer "F.Cu") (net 37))
 (segment (start 130.73 55.706) (end 133.096 53.34) (width 0.2) (layer "F.Cu") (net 39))
 (segment (start 130.73 61.39) (end 130.73 55.706) (width 0.2) (layer "F.Cu") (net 39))
 (segment (start 127 58.42) (end 128.19 59.61) (width 0.2) (layer "F.Cu") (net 28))
 (segment (start 128.19 59.61) (end 128.19 61.39) (width 0.2) (layer "F.Cu") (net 28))
 (segment (start 147.32 67.31) (end 129.275001 67.31) (width 0.2) (layer "F.Cu") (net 13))
 (segment (start 147.07 68.58) (end 147.07 67.56) (width 0.2) (layer "F.Cu") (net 13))
 (segment (start 126.92 69.665001) (end 126.92 70.69) (width 0.2) (layer "F.Cu") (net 13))
 (segment (start 156.21 65.744999) (end 154.644999 67.31) (width 0.2) (layer "F.Cu") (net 13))
 (segment (start 147.07 67.56) (end 147.32 67.31) (width 0.2) (layer "F.Cu") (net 13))
 (segment (start 156.21 64.77) (end 156.21 65.744999) (width 0.2) (layer "F.Cu") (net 13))
 (segment (start 129.275001 67.31) (end 126.92 69.665001) (width 0.2) (layer "F.Cu") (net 13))
 (segment (start 154.644999 67.31) (end 147.32 67.31) (width 0.2) (layer "F.Cu") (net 13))
 (segment (start 126.954448 72.39) (end 125.73 71.165552) (width 0.2) (layer "F.Cu") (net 11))
 (segment (start 125.73 71.165552) (end 125.73 70.214448) (width 0.2) (layer "F.Cu") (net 11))
 (segment (start 147.32 64.77) (end 147.32 66.045) (width 0.2) (layer "F.Cu") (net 11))
 (segment (start 127.514999 72.39) (end 126.954448 72.39) (width 0.2) (layer "F.Cu") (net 11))
 (segment (start 147.32 66.045) (end 154.639999 66.045) (width 0.2) (layer "F.Cu") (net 11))
 (segment (start 154.639999 66.045) (end 154.94 65.744999) (width 0.2) (layer "F.Cu") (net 11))
 (segment (start 154.94 65.744999) (end 154.94 64.77) (width 0.2) (layer "F.Cu") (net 11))
 (segment (start 129.899448 66.045) (end 147.32 66.045) (width 0.2) (layer "F.Cu") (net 11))
 (segment (start 128.19 70.69) (end 128.19 71.714999) (width 0.2) (layer "F.Cu") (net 11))
 (segment (start 128.19 71.714999) (end 127.514999 72.39) (width 0.2) (layer "F.Cu") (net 11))
 (segment (start 125.73 70.214448) (end 129.899448 66.045) (width 0.2) (layer "F.Cu") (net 11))
 (segment (start 156.09 52.19) (end 158.076346 52.19) (width 0.2) (layer "F.Cu") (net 14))
 (segment (start 158.076346 52.19) (end 158.87 52.983654) (width 0.2) (layer "F.Cu") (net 14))
 (segment (start 153.67 64.77) (end 153.67 54.61) (width 0.2) (layer "F.Cu") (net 14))
 (segment (start 153.67 54.61) (end 154.94 53.34) (width 0.2) (layer "F.Cu") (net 14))
 (segment (start 158.87 52.983654) (end 158.87 59.69) (width 0.2) (layer "F.Cu") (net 14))
 (segment (start 160.14 60.96) (end 160.985 60.96) (width 0.2) (layer "F.Cu") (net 14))
 (segment (start 154.94 53.34) (end 156.09 52.19) (width 0.2) (layer "F.Cu") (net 14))
 (segment (start 158.87 59.69) (end 160.14 60.96) (width 0.2) (layer "F.Cu") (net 14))
 (segment (start 149.86 64.77) (end 149.86 55.88) (width 0.2) (layer "F.Cu") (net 17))
 (segment (start 149.86 55.88) (end 147.32 53.34) (width 0.2) (layer "F.Cu") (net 17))
 (segment (start 152.4 64.77) (end 152.4 53.34) (width 0.2) (layer "F.Cu") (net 15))
 (segment (start 157.48 64.77) (end 157.48 53.34) (width 0.2) (layer "F.Cu") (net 12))
 (segment (start 151.13 64.77) (end 151.13 54.61) (width 0.2) (layer "F.Cu") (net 16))
 (segment (start 151.13 54.61) (end 149.86 53.34) (width 0.2) (layer "F.Cu") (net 16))
 (segment (start 162.56 60.96) (end 165.1 60.96) (width 0.2) (layer "F.Cu") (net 27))
 (segment (start 146.3 64.77) (end 143.815 64.77) (width 0.2) (layer "F.Cu") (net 10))
 (segment (start 143.815 68.58) (end 146.05 68.58) (width 0.2) (layer "F.Cu") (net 26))
 (segment (start 157.48 70.694999) (end 139.764999 88.41) (width 0.2) (layer "F.Cu") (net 22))
 (segment (start 139.764999 88.41) (end 111.18 88.41) (width 0.2) (layer "F.Cu") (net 22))
 (segment (start 157.48 69.72) (end 157.48 70.694999) (width 0.2) (layer "F.Cu") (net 22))
 (segment (start 111.18 88.41) (end 109.63 89.96) (width 0.2) (layer "F.Cu") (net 22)))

